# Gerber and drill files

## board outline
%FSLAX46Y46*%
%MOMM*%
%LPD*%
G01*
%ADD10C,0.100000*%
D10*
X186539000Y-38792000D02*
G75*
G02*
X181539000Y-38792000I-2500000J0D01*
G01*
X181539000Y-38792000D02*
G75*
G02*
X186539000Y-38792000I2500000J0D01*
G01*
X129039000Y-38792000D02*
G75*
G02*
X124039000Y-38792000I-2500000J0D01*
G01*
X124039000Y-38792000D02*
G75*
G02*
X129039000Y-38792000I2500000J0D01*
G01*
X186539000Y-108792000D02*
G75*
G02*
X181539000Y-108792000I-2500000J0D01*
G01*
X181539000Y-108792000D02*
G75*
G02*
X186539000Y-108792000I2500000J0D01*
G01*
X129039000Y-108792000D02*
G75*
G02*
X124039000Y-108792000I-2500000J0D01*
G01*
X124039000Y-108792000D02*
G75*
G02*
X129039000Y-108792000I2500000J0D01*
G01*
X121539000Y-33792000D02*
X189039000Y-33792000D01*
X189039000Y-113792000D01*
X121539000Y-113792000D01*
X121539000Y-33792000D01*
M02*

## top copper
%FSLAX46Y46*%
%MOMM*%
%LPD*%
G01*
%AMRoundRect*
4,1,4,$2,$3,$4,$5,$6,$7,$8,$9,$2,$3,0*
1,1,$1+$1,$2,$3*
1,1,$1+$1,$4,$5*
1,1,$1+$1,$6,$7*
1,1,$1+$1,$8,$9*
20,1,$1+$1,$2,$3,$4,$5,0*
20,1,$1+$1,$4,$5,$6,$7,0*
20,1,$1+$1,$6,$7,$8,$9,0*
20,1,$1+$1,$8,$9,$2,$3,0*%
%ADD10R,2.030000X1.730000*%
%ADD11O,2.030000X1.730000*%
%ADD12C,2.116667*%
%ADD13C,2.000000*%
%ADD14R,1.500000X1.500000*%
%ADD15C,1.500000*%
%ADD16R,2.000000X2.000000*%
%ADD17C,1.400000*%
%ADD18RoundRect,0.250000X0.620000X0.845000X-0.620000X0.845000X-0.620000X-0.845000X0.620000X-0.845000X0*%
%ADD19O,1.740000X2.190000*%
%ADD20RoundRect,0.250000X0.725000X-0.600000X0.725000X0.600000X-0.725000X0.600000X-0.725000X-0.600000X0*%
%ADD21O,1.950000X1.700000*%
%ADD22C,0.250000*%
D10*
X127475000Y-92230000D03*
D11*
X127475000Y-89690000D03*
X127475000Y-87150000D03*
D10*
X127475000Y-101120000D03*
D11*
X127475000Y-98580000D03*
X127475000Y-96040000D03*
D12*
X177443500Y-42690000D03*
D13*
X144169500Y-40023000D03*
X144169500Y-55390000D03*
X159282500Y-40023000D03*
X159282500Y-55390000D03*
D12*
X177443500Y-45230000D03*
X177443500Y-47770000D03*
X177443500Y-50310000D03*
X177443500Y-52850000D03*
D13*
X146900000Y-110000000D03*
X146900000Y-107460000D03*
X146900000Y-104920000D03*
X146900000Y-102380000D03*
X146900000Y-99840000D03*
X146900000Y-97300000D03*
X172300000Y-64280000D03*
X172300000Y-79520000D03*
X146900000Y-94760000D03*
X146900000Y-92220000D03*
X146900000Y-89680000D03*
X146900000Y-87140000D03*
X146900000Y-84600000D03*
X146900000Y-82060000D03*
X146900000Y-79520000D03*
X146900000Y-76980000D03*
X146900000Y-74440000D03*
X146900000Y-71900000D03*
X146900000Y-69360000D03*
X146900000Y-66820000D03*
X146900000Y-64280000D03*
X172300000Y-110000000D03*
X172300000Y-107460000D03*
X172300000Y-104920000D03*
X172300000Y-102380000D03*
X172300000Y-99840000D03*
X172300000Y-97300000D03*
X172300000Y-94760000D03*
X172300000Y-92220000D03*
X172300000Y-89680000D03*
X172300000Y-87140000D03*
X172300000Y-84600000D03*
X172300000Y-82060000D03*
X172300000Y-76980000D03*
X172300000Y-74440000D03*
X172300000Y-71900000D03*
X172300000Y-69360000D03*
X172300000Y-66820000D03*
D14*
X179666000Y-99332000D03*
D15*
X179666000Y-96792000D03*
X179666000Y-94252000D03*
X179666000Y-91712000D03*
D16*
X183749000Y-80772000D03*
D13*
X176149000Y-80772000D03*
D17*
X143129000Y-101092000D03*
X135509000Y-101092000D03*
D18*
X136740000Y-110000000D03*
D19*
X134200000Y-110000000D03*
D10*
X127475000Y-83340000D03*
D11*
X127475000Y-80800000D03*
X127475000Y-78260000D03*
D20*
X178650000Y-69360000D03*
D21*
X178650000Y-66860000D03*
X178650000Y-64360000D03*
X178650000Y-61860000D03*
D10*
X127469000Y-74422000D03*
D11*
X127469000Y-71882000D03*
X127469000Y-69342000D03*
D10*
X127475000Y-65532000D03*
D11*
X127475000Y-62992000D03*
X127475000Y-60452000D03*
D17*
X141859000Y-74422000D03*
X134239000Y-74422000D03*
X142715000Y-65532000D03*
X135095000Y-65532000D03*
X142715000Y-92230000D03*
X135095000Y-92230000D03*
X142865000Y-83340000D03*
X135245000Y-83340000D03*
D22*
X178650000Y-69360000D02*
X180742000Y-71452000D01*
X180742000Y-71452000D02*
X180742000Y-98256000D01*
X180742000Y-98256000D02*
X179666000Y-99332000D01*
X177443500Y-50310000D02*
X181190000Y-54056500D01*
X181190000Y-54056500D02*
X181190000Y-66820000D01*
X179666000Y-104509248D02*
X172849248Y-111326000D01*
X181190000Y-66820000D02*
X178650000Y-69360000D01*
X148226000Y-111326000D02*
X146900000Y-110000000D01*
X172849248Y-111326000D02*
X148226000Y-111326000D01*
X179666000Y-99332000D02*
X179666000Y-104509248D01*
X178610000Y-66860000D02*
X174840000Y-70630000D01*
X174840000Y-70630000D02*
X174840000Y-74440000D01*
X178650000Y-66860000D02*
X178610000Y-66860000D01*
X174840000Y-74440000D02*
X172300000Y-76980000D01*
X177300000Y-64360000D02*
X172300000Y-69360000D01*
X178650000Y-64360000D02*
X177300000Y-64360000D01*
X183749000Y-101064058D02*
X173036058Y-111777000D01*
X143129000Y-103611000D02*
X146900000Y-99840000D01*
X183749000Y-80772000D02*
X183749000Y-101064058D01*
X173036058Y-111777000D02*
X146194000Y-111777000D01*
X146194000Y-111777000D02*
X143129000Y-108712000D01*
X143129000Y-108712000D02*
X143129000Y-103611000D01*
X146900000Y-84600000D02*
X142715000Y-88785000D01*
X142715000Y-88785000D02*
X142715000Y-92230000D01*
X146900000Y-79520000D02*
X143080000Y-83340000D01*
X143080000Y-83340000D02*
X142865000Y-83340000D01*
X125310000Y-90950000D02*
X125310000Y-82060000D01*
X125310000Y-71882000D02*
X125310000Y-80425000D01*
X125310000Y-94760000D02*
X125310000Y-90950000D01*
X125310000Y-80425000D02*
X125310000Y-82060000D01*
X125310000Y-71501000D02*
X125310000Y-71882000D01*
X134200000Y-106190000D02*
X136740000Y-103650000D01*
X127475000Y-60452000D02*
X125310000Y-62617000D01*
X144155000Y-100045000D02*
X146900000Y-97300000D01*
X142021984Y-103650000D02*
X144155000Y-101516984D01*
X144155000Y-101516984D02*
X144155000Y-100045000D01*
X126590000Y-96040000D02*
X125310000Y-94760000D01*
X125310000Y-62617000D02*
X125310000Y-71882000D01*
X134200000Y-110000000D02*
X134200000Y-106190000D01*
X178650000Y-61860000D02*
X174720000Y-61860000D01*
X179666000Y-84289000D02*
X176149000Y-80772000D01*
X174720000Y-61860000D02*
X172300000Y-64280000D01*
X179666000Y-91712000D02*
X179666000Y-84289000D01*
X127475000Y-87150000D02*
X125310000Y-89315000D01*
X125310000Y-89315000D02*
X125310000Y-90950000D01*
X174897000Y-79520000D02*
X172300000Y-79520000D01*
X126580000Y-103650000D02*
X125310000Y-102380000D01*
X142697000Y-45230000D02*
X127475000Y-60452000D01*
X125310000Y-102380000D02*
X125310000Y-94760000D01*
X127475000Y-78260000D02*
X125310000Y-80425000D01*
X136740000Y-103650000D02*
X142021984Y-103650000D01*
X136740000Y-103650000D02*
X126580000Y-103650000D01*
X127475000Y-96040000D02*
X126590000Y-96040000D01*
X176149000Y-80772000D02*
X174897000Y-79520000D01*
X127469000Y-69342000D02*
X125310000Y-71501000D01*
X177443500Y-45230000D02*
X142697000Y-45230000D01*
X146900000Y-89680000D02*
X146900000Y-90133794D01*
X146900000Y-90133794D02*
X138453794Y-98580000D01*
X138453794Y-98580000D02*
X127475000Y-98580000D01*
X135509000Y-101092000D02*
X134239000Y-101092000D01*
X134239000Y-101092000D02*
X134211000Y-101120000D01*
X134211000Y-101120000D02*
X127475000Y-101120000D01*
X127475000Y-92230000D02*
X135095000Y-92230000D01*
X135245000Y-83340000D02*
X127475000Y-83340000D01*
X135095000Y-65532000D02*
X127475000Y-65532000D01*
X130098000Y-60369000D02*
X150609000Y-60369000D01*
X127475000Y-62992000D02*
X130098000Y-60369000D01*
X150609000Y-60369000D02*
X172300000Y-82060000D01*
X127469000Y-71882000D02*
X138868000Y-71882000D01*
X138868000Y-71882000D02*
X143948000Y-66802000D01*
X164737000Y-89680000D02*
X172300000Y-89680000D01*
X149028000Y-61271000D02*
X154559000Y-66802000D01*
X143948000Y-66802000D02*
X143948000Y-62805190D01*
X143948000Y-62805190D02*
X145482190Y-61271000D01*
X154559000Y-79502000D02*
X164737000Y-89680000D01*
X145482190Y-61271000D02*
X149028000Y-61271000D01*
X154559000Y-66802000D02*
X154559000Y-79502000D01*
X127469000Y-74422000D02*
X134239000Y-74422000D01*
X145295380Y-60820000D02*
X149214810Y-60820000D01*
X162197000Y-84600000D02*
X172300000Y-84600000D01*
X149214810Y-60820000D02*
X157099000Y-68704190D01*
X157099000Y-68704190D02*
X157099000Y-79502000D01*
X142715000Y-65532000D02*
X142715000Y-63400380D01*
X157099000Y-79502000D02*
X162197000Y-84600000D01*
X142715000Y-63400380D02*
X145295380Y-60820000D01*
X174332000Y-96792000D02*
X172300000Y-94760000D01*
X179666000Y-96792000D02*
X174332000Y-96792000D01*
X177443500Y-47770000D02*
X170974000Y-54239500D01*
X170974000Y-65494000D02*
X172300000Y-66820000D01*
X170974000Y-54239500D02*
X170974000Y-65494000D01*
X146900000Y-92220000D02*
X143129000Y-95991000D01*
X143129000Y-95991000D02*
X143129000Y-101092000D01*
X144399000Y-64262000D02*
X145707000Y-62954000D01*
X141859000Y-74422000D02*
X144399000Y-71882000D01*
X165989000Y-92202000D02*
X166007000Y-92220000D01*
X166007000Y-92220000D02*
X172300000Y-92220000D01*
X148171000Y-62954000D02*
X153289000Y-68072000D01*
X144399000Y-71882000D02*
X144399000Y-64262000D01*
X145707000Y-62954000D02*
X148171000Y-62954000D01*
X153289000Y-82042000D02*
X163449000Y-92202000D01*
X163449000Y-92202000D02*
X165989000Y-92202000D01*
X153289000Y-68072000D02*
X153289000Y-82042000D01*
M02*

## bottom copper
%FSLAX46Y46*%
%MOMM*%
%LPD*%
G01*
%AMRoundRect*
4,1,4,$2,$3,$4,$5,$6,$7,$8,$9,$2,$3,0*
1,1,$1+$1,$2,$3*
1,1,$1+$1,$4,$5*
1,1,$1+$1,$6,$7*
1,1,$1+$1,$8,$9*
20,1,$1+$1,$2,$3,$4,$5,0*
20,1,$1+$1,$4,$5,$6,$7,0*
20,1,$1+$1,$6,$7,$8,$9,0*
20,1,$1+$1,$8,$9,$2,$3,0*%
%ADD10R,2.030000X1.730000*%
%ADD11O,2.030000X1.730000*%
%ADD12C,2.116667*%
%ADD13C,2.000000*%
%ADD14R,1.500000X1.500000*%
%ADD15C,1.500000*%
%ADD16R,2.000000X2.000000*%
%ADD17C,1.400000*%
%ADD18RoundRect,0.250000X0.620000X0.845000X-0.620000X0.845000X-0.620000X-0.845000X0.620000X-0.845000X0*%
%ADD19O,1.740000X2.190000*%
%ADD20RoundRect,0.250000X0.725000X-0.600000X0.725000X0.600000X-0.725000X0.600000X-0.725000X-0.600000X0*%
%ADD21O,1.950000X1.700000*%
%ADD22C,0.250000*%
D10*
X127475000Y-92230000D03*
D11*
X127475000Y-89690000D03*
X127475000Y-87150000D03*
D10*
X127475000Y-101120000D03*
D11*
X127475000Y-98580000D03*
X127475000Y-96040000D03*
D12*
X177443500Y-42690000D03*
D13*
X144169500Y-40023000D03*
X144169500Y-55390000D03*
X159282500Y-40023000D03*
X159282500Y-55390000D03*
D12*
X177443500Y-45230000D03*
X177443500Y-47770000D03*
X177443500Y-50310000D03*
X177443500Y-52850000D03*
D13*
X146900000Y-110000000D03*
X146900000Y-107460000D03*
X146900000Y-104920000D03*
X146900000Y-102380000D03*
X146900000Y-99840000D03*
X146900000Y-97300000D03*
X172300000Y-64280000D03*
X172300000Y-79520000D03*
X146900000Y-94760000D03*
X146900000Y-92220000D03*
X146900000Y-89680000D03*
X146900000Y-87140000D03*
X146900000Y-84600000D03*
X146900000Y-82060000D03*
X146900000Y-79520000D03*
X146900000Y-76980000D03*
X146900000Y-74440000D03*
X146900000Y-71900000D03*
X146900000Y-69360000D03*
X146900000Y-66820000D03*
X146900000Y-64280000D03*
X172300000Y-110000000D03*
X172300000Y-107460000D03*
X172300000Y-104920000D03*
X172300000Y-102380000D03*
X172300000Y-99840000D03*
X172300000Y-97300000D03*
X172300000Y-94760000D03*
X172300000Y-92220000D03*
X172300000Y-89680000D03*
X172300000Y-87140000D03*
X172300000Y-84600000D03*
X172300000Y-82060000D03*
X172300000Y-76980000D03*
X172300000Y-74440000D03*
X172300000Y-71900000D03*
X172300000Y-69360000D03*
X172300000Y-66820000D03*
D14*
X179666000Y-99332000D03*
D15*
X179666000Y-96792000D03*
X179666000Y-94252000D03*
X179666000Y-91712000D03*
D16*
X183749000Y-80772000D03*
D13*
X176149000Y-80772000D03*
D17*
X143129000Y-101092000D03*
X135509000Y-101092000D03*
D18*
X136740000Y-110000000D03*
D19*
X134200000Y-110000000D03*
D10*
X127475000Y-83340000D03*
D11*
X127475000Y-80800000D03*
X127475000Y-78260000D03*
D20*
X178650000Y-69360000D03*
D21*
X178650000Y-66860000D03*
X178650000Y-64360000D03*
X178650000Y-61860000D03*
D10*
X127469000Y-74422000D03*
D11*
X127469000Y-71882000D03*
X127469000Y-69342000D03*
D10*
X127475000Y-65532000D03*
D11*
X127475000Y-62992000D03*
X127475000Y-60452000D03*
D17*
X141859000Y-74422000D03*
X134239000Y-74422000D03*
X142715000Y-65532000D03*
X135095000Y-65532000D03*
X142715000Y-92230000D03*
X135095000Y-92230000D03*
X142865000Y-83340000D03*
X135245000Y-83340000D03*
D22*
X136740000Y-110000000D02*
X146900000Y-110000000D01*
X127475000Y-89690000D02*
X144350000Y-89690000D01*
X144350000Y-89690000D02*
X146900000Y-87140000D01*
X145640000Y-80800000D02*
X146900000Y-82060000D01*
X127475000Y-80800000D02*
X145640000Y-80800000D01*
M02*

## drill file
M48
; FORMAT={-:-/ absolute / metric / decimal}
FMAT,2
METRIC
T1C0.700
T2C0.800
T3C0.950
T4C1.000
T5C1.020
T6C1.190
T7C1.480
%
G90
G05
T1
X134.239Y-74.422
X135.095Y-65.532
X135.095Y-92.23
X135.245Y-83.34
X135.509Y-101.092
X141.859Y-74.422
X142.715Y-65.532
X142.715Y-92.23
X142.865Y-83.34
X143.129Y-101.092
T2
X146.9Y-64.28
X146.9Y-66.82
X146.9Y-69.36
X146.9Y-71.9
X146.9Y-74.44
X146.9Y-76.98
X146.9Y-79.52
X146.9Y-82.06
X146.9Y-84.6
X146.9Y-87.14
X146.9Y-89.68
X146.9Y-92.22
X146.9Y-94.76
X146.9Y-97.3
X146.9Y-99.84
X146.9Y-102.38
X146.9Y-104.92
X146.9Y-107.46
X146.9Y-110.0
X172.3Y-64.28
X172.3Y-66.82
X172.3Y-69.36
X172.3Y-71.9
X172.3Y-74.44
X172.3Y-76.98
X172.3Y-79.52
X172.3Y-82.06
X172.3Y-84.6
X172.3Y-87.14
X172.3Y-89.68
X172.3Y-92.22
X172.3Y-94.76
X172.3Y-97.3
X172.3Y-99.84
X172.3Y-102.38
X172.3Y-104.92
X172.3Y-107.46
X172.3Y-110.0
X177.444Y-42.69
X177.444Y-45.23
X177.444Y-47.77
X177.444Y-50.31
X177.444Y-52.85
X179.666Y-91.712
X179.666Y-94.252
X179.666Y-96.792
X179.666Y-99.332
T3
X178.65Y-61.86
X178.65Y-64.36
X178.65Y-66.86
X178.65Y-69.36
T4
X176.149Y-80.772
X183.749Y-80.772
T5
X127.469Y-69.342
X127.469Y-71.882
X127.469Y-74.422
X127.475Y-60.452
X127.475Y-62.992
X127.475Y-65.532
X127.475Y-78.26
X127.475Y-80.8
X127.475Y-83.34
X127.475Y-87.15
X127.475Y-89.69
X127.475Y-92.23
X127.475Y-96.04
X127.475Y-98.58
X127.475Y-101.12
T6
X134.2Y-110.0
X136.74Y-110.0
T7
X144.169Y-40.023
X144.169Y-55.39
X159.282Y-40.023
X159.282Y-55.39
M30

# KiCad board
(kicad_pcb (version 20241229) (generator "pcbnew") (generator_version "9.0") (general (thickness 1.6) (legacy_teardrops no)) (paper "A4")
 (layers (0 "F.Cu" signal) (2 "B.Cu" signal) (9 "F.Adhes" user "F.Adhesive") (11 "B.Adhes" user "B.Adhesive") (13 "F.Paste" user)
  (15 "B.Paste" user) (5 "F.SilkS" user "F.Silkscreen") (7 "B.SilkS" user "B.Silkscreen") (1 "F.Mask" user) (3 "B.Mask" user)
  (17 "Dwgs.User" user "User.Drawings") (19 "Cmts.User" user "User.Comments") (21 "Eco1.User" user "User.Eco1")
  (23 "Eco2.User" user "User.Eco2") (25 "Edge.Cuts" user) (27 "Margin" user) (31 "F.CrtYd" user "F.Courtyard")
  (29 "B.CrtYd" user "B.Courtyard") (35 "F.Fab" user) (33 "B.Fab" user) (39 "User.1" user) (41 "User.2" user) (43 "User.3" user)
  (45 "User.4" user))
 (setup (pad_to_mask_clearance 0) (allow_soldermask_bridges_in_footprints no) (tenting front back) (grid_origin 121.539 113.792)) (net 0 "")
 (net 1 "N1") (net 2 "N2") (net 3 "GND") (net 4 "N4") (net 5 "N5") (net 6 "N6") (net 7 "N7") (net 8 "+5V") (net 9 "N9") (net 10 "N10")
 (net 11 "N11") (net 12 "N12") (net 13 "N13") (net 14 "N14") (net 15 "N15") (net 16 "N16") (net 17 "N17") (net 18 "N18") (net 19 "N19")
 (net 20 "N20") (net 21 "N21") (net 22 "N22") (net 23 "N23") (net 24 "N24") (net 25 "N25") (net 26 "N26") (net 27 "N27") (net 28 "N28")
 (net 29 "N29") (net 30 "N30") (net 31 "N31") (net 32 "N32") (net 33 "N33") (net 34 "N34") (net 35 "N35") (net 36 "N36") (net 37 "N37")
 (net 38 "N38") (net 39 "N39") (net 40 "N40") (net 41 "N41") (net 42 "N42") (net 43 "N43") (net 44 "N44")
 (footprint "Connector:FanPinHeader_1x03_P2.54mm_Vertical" (layer "F.Cu") (at 127.475 92.23 90)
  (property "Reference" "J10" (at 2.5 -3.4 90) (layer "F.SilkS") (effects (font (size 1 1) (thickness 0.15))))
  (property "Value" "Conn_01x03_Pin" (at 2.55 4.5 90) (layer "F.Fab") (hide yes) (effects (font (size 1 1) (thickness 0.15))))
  (pad "1" thru_hole rect (at 0 0 180) (size 2.03 1.73) (drill 1.02) (layers "*.Cu" "*.Mask") (remove_unused_layers no) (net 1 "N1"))
  (pad "2" thru_hole oval (at 2.54 0 180) (size 2.03 1.73) (drill 1.02) (layers "*.Cu" "*.Mask") (remove_unused_layers no) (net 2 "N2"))
  (pad "3" thru_hole oval (at 5.08 0 180) (size 2.03 1.73) (drill 1.02) (layers "*.Cu" "*.Mask") (remove_unused_layers no) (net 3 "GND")))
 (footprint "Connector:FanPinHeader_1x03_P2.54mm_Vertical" (layer "F.Cu") (at 127.475 101.12 90)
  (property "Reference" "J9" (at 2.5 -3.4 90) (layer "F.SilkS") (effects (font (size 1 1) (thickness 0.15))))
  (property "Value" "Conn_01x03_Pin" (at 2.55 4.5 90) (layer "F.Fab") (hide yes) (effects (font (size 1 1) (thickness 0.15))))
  (pad "1" thru_hole rect (at 0 0 180) (size 2.03 1.73) (drill 1.02) (layers "*.Cu" "*.Mask") (remove_unused_layers no) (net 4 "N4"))
  (pad "2" thru_hole oval (at 2.54 0 180) (size 2.03 1.73) (drill 1.02) (layers "*.Cu" "*.Mask") (remove_unused_layers no) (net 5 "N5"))
  (pad "3" thru_hole oval (at 5.08 0 180) (size 2.03 1.73) (drill 1.02) (layers "*.Cu" "*.Mask") (remove_unused_layers no) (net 3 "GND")))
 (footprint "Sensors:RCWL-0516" (layer "F.Cu") (at 164.7435 47.77)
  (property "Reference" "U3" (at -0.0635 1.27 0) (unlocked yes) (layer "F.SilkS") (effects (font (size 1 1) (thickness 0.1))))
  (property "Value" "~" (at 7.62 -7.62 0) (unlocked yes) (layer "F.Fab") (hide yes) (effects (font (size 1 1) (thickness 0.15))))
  (pad "1" thru_hole circle (at 12.7 -5.08 180) (size 2.116667 2.116667) (drill 0.8) (layers "*.Cu" "*.Mask") (remove_unused_layers no)
   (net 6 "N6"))
  (pad "2" thru_hole circle (at -20.574 -7.747 180) (size 2 2) (drill 1.48) (layers "*.Cu" "*.Mask") (remove_unused_layers no) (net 3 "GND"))
  (pad "2" thru_hole circle (at -20.574 7.62 180) (size 2 2) (drill 1.48) (layers "*.Cu" "*.Mask") (remove_unused_layers no) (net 3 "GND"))
  (pad "2" thru_hole circle (at -5.461 -7.747 180) (size 2 2) (drill 1.48) (layers "*.Cu" "*.Mask") (remove_unused_layers no) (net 3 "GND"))
  (pad "2" thru_hole circle (at -5.461 7.62 180) (size 2 2) (drill 1.48) (layers "*.Cu" "*.Mask") (remove_unused_layers no) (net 3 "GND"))
  (pad "2" thru_hole circle (at 12.7 -2.54 180) (size 2.116667 2.116667) (drill 0.8) (layers "*.Cu" "*.Mask") (remove_unused_layers no)
   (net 3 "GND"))
  (pad "3" thru_hole circle (at 12.7 0 180) (size 2.116667 2.116667) (drill 0.8) (layers "*.Cu" "*.Mask") (remove_unused_layers no)
   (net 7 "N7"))
  (pad "4" thru_hole circle (at 12.7 2.54 180) (size 2.116667 2.116667) (drill 0.8) (layers "*.Cu" "*.Mask") (remove_unused_layers no)
   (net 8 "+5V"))
  (pad "5" thru_hole circle (at 12.7 5.08 180) (size 2.116667 2.116667) (drill 0.8) (layers "*.Cu" "*.Mask") (remove_unused_layers no)
   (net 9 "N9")))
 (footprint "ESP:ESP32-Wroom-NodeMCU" (layer "F.Cu") (at 146.9 110)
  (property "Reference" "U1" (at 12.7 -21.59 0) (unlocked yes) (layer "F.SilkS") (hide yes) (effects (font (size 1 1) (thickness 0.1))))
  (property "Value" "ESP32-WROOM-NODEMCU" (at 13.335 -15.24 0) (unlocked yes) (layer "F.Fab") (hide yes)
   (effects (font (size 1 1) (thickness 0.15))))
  (pad "1" thru_hole circle (at 0 0) (size 2 2) (drill 0.8) (layers "*.Cu" "*.Mask") (remove_unused_layers no) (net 8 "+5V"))
  (pad "2" thru_hole circle (at 0 -2.54) (size 2 2) (drill 0.8) (layers "*.Cu" "*.Mask") (remove_unused_layers no) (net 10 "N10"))
  (pad "3" thru_hole circle (at 0 -5.08) (size 2 2) (drill 0.8) (layers "*.Cu" "*.Mask") (remove_unused_layers no) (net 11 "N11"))
  (pad "4" thru_hole circle (at 0 -7.62) (size 2 2) (drill 0.8) (layers "*.Cu" "*.Mask") (remove_unused_layers no) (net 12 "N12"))
  (pad "5" thru_hole circle (at 0 -10.16) (size 2 2) (drill 0.8) (layers "*.Cu" "*.Mask") (remove_unused_layers no) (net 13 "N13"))
  (pad "6" thru_hole circle (at 0 -12.7) (size 2 2) (drill 0.8) (layers "*.Cu" "*.Mask") (remove_unused_layers no) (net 3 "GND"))
  (pad "6" thru_hole circle (at 25.4 -45.72) (size 2 2) (drill 0.8) (layers "*.Cu" "*.Mask") (remove_unused_layers no) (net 3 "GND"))
  (pad "6" thru_hole circle (at 25.4 -30.48) (size 2 2) (drill 0.8) (layers "*.Cu" "*.Mask") (remove_unused_layers no) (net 3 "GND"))
  (pad "7" thru_hole circle (at 0 -15.24) (size 2 2) (drill 0.8) (layers "*.Cu" "*.Mask") (remove_unused_layers no) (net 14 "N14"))
  (pad "8" thru_hole circle (at 0 -17.78) (size 2 2) (drill 0.8) (layers "*.Cu" "*.Mask") (remove_unused_layers no) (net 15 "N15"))
  (pad "9" thru_hole circle (at 0 -20.32) (size 2 2) (drill 0.8) (layers "*.Cu" "*.Mask") (remove_unused_layers no) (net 5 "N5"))
  (pad "10" thru_hole circle (at 0 -22.86) (size 2 2) (drill 0.8) (layers "*.Cu" "*.Mask") (remove_unused_layers no) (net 2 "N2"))
  (pad "11" thru_hole circle (at 0 -25.4) (size 2 2) (drill 0.8) (layers "*.Cu" "*.Mask") (remove_unused_layers no) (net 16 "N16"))
  (pad "12" thru_hole circle (at 0 -27.94) (size 2 2) (drill 0.8) (layers "*.Cu" "*.Mask") (remove_unused_layers no) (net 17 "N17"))
  (pad "13" thru_hole circle (at 0 -30.48) (size 2 2) (drill 0.8) (layers "*.Cu" "*.Mask") (remove_unused_layers no) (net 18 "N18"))
  (pad "14" thru_hole circle (at 0 -33.02) (size 2 2) (drill 0.8) (layers "*.Cu" "*.Mask") (remove_unused_layers no) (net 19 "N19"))
  (pad "15" thru_hole circle (at 0 -35.56) (size 2 2) (drill 0.8) (layers "*.Cu" "*.Mask") (remove_unused_layers no) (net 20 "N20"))
  (pad "16" thru_hole circle (at 0 -38.1) (size 2 2) (drill 0.8) (layers "*.Cu" "*.Mask") (remove_unused_layers no) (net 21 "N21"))
  (pad "17" thru_hole circle (at 0 -40.64) (size 2 2) (drill 0.8) (layers "*.Cu" "*.Mask") (remove_unused_layers no) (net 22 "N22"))
  (pad "18" thru_hole circle (at 0 -43.18) (size 2 2) (drill 0.8) (layers "*.Cu" "*.Mask") (remove_unused_layers no) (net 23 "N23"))
  (pad "19" thru_hole circle (at 0 -45.72) (size 2 2) (drill 0.8) (layers "*.Cu" "*.Mask") (remove_unused_layers no) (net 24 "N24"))
  (pad "20" thru_hole circle (at 25.4 0) (size 2 2) (drill 0.8) (layers "*.Cu" "*.Mask") (remove_unused_layers no) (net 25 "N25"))
  (pad "21" thru_hole circle (at 25.4 -2.54) (size 2 2) (drill 0.8) (layers "*.Cu" "*.Mask") (remove_unused_layers no) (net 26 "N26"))
  (pad "22" thru_hole circle (at 25.4 -5.08) (size 2 2) (drill 0.8) (layers "*.Cu" "*.Mask") (remove_unused_layers no) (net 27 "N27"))
  (pad "23" thru_hole circle (at 25.4 -7.62) (size 2 2) (drill 0.8) (layers "*.Cu" "*.Mask") (remove_unused_layers no) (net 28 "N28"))
  (pad "24" thru_hole circle (at 25.4 -10.16) (size 2 2) (drill 0.8) (layers "*.Cu" "*.Mask") (remove_unused_layers no) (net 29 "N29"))
  (pad "25" thru_hole circle (at 25.4 -12.7) (size 2 2) (drill 0.8) (layers "*.Cu" "*.Mask") (remove_unused_layers no) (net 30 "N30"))
  (pad "26" thru_hole circle (at 25.4 -15.24) (size 2 2) (drill 0.8) (layers "*.Cu" "*.Mask") (remove_unused_layers no) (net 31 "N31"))
  (pad "27" thru_hole circle (at 25.4 -17.78) (size 2 2) (drill 0.8) (layers "*.Cu" "*.Mask") (remove_unused_layers no) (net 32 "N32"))
  (pad "28" thru_hole circle (at 25.4 -20.32) (size 2 2) (drill 0.8) (layers "*.Cu" "*.Mask") (remove_unused_layers no) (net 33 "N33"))
  (pad "29" thru_hole circle (at 25.4 -22.86) (size 2 2) (drill 0.8) (layers "*.Cu" "*.Mask") (remove_unused_layers no) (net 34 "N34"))
  (pad "30" thru_hole circle (at 25.4 -25.4) (size 2 2) (drill 0.8) (layers "*.Cu" "*.Mask") (remove_unused_layers no) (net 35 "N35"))
  (pad "31" thru_hole circle (at 25.4 -27.94) (size 2 2) (drill 0.8) (layers "*.Cu" "*.Mask") (remove_unused_layers no) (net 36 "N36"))
  (pad "33" thru_hole circle (at 25.4 -33.02) (size 2 2) (drill 0.8) (layers "*.Cu" "*.Mask") (remove_unused_layers no) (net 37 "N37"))
  (pad "34" thru_hole circle (at 25.4 -35.56) (size 2 2) (drill 0.8) (layers "*.Cu" "*.Mask") (remove_unused_layers no) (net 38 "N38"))
  (pad "35" thru_hole circle (at 25.4 -38.1) (size 2 2) (drill 0.8) (layers "*.Cu" "*.Mask") (remove_unused_layers no) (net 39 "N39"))
  (pad "36" thru_hole circle (at 25.4 -40.64) (size 2 2) (drill 0.8) (layers "*.Cu" "*.Mask") (remove_unused_layers no) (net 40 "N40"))
  (pad "37" thru_hole circle (at 25.4 -43.18) (size 2 2) (drill 0.8) (layers "*.Cu" "*.Mask") (remove_unused_layers no) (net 7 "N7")))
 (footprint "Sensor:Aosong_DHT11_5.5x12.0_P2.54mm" (layer "F.Cu") (at 179.666 99.332 180)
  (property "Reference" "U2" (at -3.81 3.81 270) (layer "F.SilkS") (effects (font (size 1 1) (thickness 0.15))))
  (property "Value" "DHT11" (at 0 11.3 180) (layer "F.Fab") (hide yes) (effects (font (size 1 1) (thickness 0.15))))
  (pad "1" thru_hole rect (at 0 0 180) (size 1.5 1.5) (drill 0.8) (layers "*.Cu" "*.Mask") (remove_unused_layers no) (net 8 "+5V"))
  (pad "2" thru_hole circle (at 0 2.54 180) (size 1.5 1.5) (drill 0.8) (layers "*.Cu" "*.Mask") (remove_unused_layers no) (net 31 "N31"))
  (pad "3" thru_hole circle (at 0 5.08 180) (size 1.5 1.5) (drill 0.8) (layers "*.Cu" "*.Mask") (remove_unused_layers no) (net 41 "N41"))
  (pad "4" thru_hole circle (at 0 7.62 180) (size 1.5 1.5) (drill 0.8) (layers "*.Cu" "*.Mask") (remove_unused_layers no) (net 3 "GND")))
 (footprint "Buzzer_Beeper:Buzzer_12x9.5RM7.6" (layer "F.Cu") (at 183.749 80.772 180)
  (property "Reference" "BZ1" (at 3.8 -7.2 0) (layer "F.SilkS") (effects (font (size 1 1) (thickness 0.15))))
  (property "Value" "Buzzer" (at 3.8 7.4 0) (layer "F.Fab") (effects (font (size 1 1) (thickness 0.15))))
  (pad "1" thru_hole rect (at 0 0 180) (size 2 2) (drill 1) (layers "*.Cu" "*.Mask") (remove_unused_layers no) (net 13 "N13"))
  (pad "2" thru_hole circle (at 7.6 0 180) (size 2 2) (drill 1) (layers "*.Cu" "*.Mask") (remove_unused_layers no) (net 3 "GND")))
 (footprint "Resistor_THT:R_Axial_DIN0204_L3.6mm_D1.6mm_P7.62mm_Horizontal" (layer "F.Cu") (at 143.129 101.092 180)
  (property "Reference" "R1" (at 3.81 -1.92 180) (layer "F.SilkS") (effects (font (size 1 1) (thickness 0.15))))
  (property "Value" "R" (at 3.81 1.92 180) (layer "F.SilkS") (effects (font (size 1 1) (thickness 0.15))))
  (pad "1" thru_hole circle (at 0 0 180) (size 1.4 1.4) (drill 0.7) (layers "*.Cu" "*.Mask") (remove_unused_layers no) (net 15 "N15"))
  (pad "2" thru_hole circle (at 7.62 0 180) (size 1.4 1.4) (drill 0.7) (layers "*.Cu" "*.Mask") (remove_unused_layers no) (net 4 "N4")))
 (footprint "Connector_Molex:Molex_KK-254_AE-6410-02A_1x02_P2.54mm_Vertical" (layer "F.Cu") (at 136.74 110 180)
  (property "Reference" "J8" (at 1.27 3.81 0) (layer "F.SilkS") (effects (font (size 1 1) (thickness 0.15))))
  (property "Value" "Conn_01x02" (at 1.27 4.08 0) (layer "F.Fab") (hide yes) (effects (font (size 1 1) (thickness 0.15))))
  (pad "1" thru_hole roundrect (at 0 0 180) (size 1.74 2.19) (drill 1.19) (layers "*.Cu" "*.Mask") (remove_unused_layers no)
   (roundrect_rratio 0.143678) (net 8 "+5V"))
  (pad "2" thru_hole oval (at 2.54 0 180) (size 1.74 2.19) (drill 1.19) (layers "*.Cu" "*.Mask") (remove_unused_layers no) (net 3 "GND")))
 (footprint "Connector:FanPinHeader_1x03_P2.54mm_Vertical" (layer "F.Cu") (at 127.475 83.34 90)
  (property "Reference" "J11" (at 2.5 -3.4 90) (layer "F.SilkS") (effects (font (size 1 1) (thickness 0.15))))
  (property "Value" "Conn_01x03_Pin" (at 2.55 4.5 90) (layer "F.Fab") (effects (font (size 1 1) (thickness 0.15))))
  (pad "1" thru_hole rect (at 0 0 180) (size 2.03 1.73) (drill 1.02) (layers "*.Cu" "*.Mask") (remove_unused_layers no) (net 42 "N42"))
  (pad "2" thru_hole oval (at 2.54 0 180) (size 2.03 1.73) (drill 1.02) (layers "*.Cu" "*.Mask") (remove_unused_layers no) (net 17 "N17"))
  (pad "3" thru_hole oval (at 5.08 0 180) (size 2.03 1.73) (drill 1.02) (layers "*.Cu" "*.Mask") (remove_unused_layers no) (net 3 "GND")))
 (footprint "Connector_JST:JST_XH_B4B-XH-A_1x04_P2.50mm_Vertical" (layer "F.Cu") (at 178.65 69.36 90)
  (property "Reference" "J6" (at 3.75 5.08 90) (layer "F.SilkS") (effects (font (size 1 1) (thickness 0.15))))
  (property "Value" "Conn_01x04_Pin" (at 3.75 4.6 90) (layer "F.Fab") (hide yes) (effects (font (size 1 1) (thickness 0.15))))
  (pad "1" thru_hole roundrect (at 0 0 90) (size 1.7 1.95) (drill 0.95) (layers "*.Cu" "*.Mask") (remove_unused_layers no)
   (roundrect_rratio 0.147059) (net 8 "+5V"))
  (pad "2" thru_hole oval (at 2.5 0 90) (size 1.7 1.95) (drill 0.95) (layers "*.Cu" "*.Mask") (remove_unused_layers no) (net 37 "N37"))
  (pad "3" thru_hole oval (at 5 0 90) (size 1.7 1.95) (drill 0.95) (layers "*.Cu" "*.Mask") (remove_unused_layers no) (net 40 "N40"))
  (pad "4" thru_hole oval (at 7.5 0 90) (size 1.7 1.95) (drill 0.95) (layers "*.Cu" "*.Mask") (remove_unused_layers no) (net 3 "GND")))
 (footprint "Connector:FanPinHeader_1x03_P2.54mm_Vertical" (layer "F.Cu") (at 127.469 74.422 90)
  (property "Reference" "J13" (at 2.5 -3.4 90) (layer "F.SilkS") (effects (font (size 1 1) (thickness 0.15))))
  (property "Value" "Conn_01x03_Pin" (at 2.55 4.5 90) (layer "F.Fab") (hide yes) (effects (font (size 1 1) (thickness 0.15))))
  (pad "1" thru_hole rect (at 0 0 180) (size 2.03 1.73) (drill 1.02) (layers "*.Cu" "*.Mask") (remove_unused_layers no) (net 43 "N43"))
  (pad "2" thru_hole oval (at 2.54 0 180) (size 2.03 1.73) (drill 1.02) (layers "*.Cu" "*.Mask") (remove_unused_layers no) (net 33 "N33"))
  (pad "3" thru_hole oval (at 5.08 0 180) (size 2.03 1.73) (drill 1.02) (layers "*.Cu" "*.Mask") (remove_unused_layers no) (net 3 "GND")))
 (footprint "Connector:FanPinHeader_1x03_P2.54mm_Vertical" (layer "F.Cu") (at 127.475 65.532 90)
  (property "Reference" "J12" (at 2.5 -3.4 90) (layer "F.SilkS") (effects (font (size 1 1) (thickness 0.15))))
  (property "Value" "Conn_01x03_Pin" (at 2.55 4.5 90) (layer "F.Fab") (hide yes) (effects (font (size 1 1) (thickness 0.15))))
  (pad "1" thru_hole rect (at 0 0 180) (size 2.03 1.73) (drill 1.02) (layers "*.Cu" "*.Mask") (remove_unused_layers no) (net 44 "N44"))
  (pad "2" thru_hole oval (at 2.54 0 180) (size 2.03 1.73) (drill 1.02) (layers "*.Cu" "*.Mask") (remove_unused_layers no) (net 36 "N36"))
  (pad "3" thru_hole oval (at 5.08 0 180) (size 2.03 1.73) (drill 1.02) (layers "*.Cu" "*.Mask") (remove_unused_layers no) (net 3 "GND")))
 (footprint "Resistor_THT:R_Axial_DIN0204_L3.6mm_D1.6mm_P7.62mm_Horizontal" (layer "F.Cu") (at 141.859 74.422 180)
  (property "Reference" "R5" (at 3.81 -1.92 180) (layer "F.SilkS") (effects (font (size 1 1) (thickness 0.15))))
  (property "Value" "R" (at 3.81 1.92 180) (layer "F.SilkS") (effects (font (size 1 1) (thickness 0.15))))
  (pad "1" thru_hole circle (at 0 0 180) (size 1.4 1.4) (drill 0.7) (layers "*.Cu" "*.Mask") (remove_unused_layers no) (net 32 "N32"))
  (pad "2" thru_hole circle (at 7.62 0 180) (size 1.4 1.4) (drill 0.7) (layers "*.Cu" "*.Mask") (remove_unused_layers no) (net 43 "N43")))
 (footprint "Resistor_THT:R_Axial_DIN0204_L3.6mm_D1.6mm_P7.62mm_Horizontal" (layer "F.Cu") (at 142.715 65.532 180)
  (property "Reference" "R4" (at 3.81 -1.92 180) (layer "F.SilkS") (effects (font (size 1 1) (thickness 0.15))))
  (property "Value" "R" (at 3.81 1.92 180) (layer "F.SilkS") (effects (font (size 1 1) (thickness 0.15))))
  (pad "1" thru_hole circle (at 0 0 180) (size 1.4 1.4) (drill 0.7) (layers "*.Cu" "*.Mask") (remove_unused_layers no) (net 35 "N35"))
  (pad "2" thru_hole circle (at 7.62 0 180) (size 1.4 1.4) (drill 0.7) (layers "*.Cu" "*.Mask") (remove_unused_layers no) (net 44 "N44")))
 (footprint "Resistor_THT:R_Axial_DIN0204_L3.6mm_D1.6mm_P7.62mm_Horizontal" (layer "F.Cu") (at 142.715 92.23 180)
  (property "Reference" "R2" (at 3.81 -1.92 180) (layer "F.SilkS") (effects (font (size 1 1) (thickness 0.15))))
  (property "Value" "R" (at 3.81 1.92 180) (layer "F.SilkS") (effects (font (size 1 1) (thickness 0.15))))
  (pad "1" thru_hole circle (at 0 0 180) (size 1.4 1.4) (drill 0.7) (layers "*.Cu" "*.Mask") (remove_unused_layers no) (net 16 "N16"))
  (pad "2" thru_hole circle (at 7.62 0 180) (size 1.4 1.4) (drill 0.7) (layers "*.Cu" "*.Mask") (remove_unused_layers no) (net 1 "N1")))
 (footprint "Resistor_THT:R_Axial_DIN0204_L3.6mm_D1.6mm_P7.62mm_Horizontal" (layer "F.Cu") (at 142.865 83.34 180)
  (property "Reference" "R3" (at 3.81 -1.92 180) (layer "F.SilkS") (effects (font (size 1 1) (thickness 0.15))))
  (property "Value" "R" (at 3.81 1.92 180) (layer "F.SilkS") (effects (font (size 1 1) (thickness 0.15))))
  (pad "1" thru_hole circle (at 0 0 180) (size 1.4 1.4) (drill 0.7) (layers "*.Cu" "*.Mask") (remove_unused_layers no) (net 18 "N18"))
  (pad "2" thru_hole circle (at 7.62 0 180) (size 1.4 1.4) (drill 0.7) (layers "*.Cu" "*.Mask") (remove_unused_layers no) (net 42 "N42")))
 (gr_circle (center 184.039 38.792) (end 184.039 41.292) (stroke (width 0.1) (type default)) (fill no) (layer "Edge.Cuts"))
 (gr_circle (center 126.539 38.792) (end 126.539 41.292) (stroke (width 0.1) (type default)) (fill no) (layer "Edge.Cuts"))
 (gr_circle (center 184.039 108.792) (end 186.539 108.792) (stroke (width 0.1) (type default)) (fill no) (layer "Edge.Cuts"))
 (gr_circle (center 126.539 108.792) (end 126.539 111.292) (stroke (width 0.1) (type default)) (fill no) (layer "Edge.Cuts"))
 (gr_rect (start 121.539 33.792) (end 189.039 113.792) (stroke (width 0.1) (type default)) (fill no) (layer "Edge.Cuts"))
 (segment (start 178.65 69.36) (end 180.742 71.452) (width 0.25) (layer "F.Cu") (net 8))
 (segment (start 180.742 71.452) (end 180.742 98.256) (width 0.25) (layer "F.Cu") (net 8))
 (segment (start 180.742 98.256) (end 179.666 99.332) (width 0.25) (layer "F.Cu") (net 8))
 (segment (start 177.4435 50.31) (end 181.19 54.0565) (width 0.25) (layer "F.Cu") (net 8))
 (segment (start 181.19 54.0565) (end 181.19 66.82) (width 0.25) (layer "F.Cu") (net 8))
 (segment (start 179.666 104.509248) (end 172.849248 111.326) (width 0.25) (layer "F.Cu") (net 8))
 (segment (start 181.19 66.82) (end 178.65 69.36) (width 0.25) (layer "F.Cu") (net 8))
 (segment (start 148.226 111.326) (end 146.9 110) (width 0.25) (layer "F.Cu") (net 8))
 (segment (start 172.849248 111.326) (end 148.226 111.326) (width 0.25) (layer "F.Cu") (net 8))
 (segment (start 179.666 99.332) (end 179.666 104.509248) (width 0.25) (layer "F.Cu") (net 8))
 (segment (start 136.74 110) (end 146.9 110) (width 0.25) (layer "B.Cu") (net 8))
 (segment (start 178.61 66.86) (end 174.84 70.63) (width 0.25) (layer "F.Cu") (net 37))
 (segment (start 174.84 70.63) (end 174.84 74.44) (width 0.25) (layer "F.Cu") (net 37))
 (segment (start 178.65 66.86) (end 178.61 66.86) (width 0.25) (layer "F.Cu") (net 37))
 (segment (start 174.84 74.44) (end 172.3 76.98) (width 0.25) (layer "F.Cu") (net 37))
 (segment (start 177.3 64.36) (end 172.3 69.36) (width 0.25) (layer "F.Cu") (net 40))
 (segment (start 178.65 64.36) (end 177.3 64.36) (width 0.25) (layer "F.Cu") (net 40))
 (segment (start 183.749 101.064058) (end 173.036058 111.777) (width 0.25) (layer "F.Cu") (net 13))
 (segment (start 143.129 103.611) (end 146.9 99.84) (width 0.25) (layer "F.Cu") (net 13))
 (segment (start 183.749 80.772) (end 183.749 101.064058) (width 0.25) (layer "F.Cu") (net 13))
 (segment (start 173.036058 111.777) (end 146.194 111.777) (width 0.25) (layer "F.Cu") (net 13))
 (segment (start 146.194 111.777) (end 143.129 108.712) (width 0.25) (layer "F.Cu") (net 13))
 (segment (start 143.129 108.712) (end 143.129 103.611) (width 0.25) (layer "F.Cu") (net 13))
 (segment (start 146.9 84.6) (end 142.715 88.785) (width 0.25) (layer "F.Cu") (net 16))
 (segment (start 142.715 88.785) (end 142.715 92.23) (width 0.25) (layer "F.Cu") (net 16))
 (segment (start 146.9 79.52) (end 143.08 83.34) (width 0.25) (layer "F.Cu") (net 18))
 (segment (start 143.08 83.34) (end 142.865 83.34) (width 0.25) (layer "F.Cu") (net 18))
 (segment (start 125.31 90.95) (end 125.31 82.06) (width 0.25) (layer "F.Cu") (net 3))
 (segment (start 125.31 71.882) (end 125.31 80.425) (width 0.25) (layer "F.Cu") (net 3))
 (segment (start 125.31 94.76) (end 125.31 90.95) (width 0.25) (layer "F.Cu") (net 3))
 (segment (start 125.31 80.425) (end 125.31 82.06) (width 0.25) (layer "F.Cu") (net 3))
 (segment (start 125.31 71.501) (end 125.31 71.882) (width 0.25) (layer "F.Cu") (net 3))
 (segment (start 134.2 106.19) (end 136.74 103.65) (width 0.25) (layer "F.Cu") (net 3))
 (segment (start 127.475 60.452) (end 125.31 62.617) (width 0.25) (layer "F.Cu") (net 3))
 (segment (start 144.155 100.045) (end 146.9 97.3) (width 0.25) (layer "F.Cu") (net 3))
 (segment (start 142.021984 103.65) (end 144.155 101.516984) (width 0.25) (layer "F.Cu") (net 3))
 (segment (start 144.155 101.516984) (end 144.155 100.045) (width 0.25) (layer "F.Cu") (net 3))
 (segment (start 126.59 96.04) (end 125.31 94.76) (width 0.25) (layer "F.Cu") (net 3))
 (segment (start 125.31 62.617) (end 125.31 71.882) (width 0.25) (layer "F.Cu") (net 3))
 (segment (start 134.2 110) (end 134.2 106.19) (width 0.25) (layer "F.Cu") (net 3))
 (segment (start 178.65 61.86) (end 174.72 61.86) (width 0.25) (layer "F.Cu") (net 3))
 (segment (start 179.666 84.289) (end 176.149 80.772) (width 0.25) (layer "F.Cu") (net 3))
 (segment (start 174.72 61.86) (end 172.3 64.28) (width 0.25) (layer "F.Cu") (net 3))
 (segment (start 179.666 91.712) (end 179.666 84.289) (width 0.25) (layer "F.Cu") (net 3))
 (segment (start 127.475 87.15) (end 125.31 89.315) (width 0.25) (layer "F.Cu") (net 3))
 (segment (start 125.31 89.315) (end 125.31 90.95) (width 0.25) (layer "F.Cu") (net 3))
 (segment (start 174.897 79.52) (end 172.3 79.52) (width 0.25) (layer "F.Cu") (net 3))
 (segment (start 126.58 103.65) (end 125.31 102.38) (width 0.25) (layer "F.Cu") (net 3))
 (segment (start 142.697 45.23) (end 127.475 60.452) (width 0.25) (layer "F.Cu") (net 3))
 (segment (start 125.31 102.38) (end 125.31 94.76) (width 0.25) (layer "F.Cu") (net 3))
 (segment (start 127.475 78.26) (end 125.31 80.425) (width 0.25) (layer "F.Cu") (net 3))
 (segment (start 136.74 103.65) (end 142.021984 103.65) (width 0.25) (layer "F.Cu") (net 3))
 (segment (start 136.74 103.65) (end 126.58 103.65) (width 0.25) (layer "F.Cu") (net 3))
 (segment (start 127.475 96.04) (end 126.59 96.04) (width 0.25) (layer "F.Cu") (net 3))
 (segment (start 176.149 80.772) (end 174.897 79.52) (width 0.25) (layer "F.Cu") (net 3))
 (segment (start 127.469 69.342) (end 125.31 71.501) (width 0.25) (layer "F.Cu") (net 3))
 (segment (start 177.4435 45.23) (end 142.697 45.23) (width 0.25) (layer "F.Cu") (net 3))
 (segment (start 146.9 89.68) (end 146.9 90.133794) (width 0.25) (layer "F.Cu") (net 5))
 (segment (start 146.9 90.133794) (end 138.453794 98.58) (width 0.25) (layer "F.Cu") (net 5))
 (segment (start 138.453794 98.58) (end 127.475 98.58) (width 0.25) (layer "F.Cu") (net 5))
 (segment (start 135.509 101.092) (end 134.239 101.092) (width 0.25) (layer "F.Cu") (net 4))
 (segment (start 134.239 101.092) (end 134.211 101.12) (width 0.25) (layer "F.Cu") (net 4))
 (segment (start 134.211 101.12) (end 127.475 101.12) (width 0.25) (layer "F.Cu") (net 4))
 (segment (start 127.475 92.23) (end 135.095 92.23) (width 0.25) (layer "F.Cu") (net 1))
 (segment (start 127.475 89.69) (end 144.35 89.69) (width 0.25) (layer "B.Cu") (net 2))
 (segment (start 144.35 89.69) (end 146.9 87.14) (width 0.25) (layer "B.Cu") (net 2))
 (segment (start 135.245 83.34) (end 127.475 83.34) (width 0.25) (layer "F.Cu") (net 42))
 (segment (start 145.64 80.8) (end 146.9 82.06) (width 0.25) (layer "B.Cu") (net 17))
 (segment (start 127.475 80.8) (end 145.64 80.8) (width 0.25) (layer "B.Cu") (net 17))
 (segment (start 135.095 65.532) (end 127.475 65.532) (width 0.25) (layer "F.Cu") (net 44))
 (segment (start 130.098 60.369) (end 150.609 60.369) (width 0.25) (layer "F.Cu") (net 36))
 (segment (start 127.475 62.992) (end 130.098 60.369) (width 0.25) (layer "F.Cu") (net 36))
 (segment (start 150.609 60.369) (end 172.3 82.06) (width 0.25) (layer "F.Cu") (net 36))
 (segment (start 127.469 71.882) (end 138.868 71.882) (width 0.25) (layer "F.Cu") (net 33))
 (segment (start 138.868 71.882) (end 143.948 66.802) (width 0.25) (layer "F.Cu") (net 33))
 (segment (start 164.737 89.68) (end 172.3 89.68) (width 0.25) (layer "F.Cu") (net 33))
 (segment (start 149.028 61.271) (end 154.559 66.802) (width 0.25) (layer "F.Cu") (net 33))
 (segment (start 143.948 66.802) (end 143.948 62.80519) (width 0.25) (layer "F.Cu") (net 33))
 (segment (start 143.948 62.80519) (end 145.48219 61.271) (width 0.25) (layer "F.Cu") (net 33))
 (segment (start 154.559 79.502) (end 164.737 89.68) (width 0.25) (layer "F.Cu") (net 33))
 (segment (start 145.48219 61.271) (end 149.028 61.271) (width 0.25) (layer "F.Cu") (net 33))
 (segment (start 154.559 66.802) (end 154.559 79.502) (width 0.25) (layer "F.Cu") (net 33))
 (segment (start 127.469 74.422) (end 134.239 74.422) (width 0.25) (layer "F.Cu") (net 43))
 (segment (start 145.29538 60.82) (end 149.21481 60.82) (width 0.25) (layer "F.Cu") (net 35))
 (segment (start 162.197 84.6) (end 172.3 84.6) (width 0.25) (layer "F.Cu") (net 35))
 (segment (start 149.21481 60.82) (end 157.099 68.70419) (width 0.25) (layer "F.Cu") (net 35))
 (segment (start 157.099 68.70419) (end 157.099 79.502) (width 0.25) (layer "F.Cu") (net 35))
 (segment (start 142.715 65.532) (end 142.715 63.40038) (width 0.25) (layer "F.Cu") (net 35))
 (segment (start 157.099 79.502) (end 162.197 84.6) (width 0.25) (layer "F.Cu") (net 35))
 (segment (start 142.715 63.40038) (end 145.29538 60.82) (width 0.25) (layer "F.Cu") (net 35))
 (segment (start 174.332 96.792) (end 172.3 94.76) (width 0.25) (layer "F.Cu") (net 31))
 (segment (start 179.666 96.792) (end 174.332 96.792) (width 0.25) (layer "F.Cu") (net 31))
 (segment (start 177.4435 47.77) (end 170.974 54.2395) (width 0.25) (layer "F.Cu") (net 7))
 (segment (start 170.974 65.494) (end 172.3 66.82) (width 0.25) (layer "F.Cu") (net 7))
 (segment (start 170.974 54.2395) (end 170.974 65.494) (width 0.25) (layer "F.Cu") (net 7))
 (segment (start 146.9 92.22) (end 143.129 95.991) (width 0.25) (layer "F.Cu") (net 15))
 (segment (start 143.129 95.991) (end 143.129 101.092) (width 0.25) (layer "F.Cu") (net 15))
 (segment (start 144.399 64.262) (end 145.707 62.954) (width 0.25) (layer "F.Cu") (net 32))
 (segment (start 141.859 74.422) (end 144.399 71.882) (width 0.25) (layer "F.Cu") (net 32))
 (segment (start 165.989 92.202) (end 166.007 92.22) (width 0.25) (layer "F.Cu") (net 32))
 (segment (start 166.007 92.22) (end 172.3 92.22) (width 0.25) (layer "F.Cu") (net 32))
 (segment (start 148.171 62.954) (end 153.289 68.072) (width 0.25) (layer "F.Cu") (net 32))
 (segment (start 144.399 71.882) (end 144.399 64.262) (width 0.25) (layer "F.Cu") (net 32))
 (segment (start 145.707 62.954) (end 148.171 62.954) (width 0.25) (layer "F.Cu") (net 32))
 (segment (start 153.289 82.042) (end 163.449 92.202) (width 0.25) (layer "F.Cu") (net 32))
 (segment (start 163.449 92.202) (end 165.989 92.202) (width 0.25) (layer "F.Cu") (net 32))
 (segment (start 153.289 68.072) (end 153.289 82.042) (width 0.25) (layer "F.Cu") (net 32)))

